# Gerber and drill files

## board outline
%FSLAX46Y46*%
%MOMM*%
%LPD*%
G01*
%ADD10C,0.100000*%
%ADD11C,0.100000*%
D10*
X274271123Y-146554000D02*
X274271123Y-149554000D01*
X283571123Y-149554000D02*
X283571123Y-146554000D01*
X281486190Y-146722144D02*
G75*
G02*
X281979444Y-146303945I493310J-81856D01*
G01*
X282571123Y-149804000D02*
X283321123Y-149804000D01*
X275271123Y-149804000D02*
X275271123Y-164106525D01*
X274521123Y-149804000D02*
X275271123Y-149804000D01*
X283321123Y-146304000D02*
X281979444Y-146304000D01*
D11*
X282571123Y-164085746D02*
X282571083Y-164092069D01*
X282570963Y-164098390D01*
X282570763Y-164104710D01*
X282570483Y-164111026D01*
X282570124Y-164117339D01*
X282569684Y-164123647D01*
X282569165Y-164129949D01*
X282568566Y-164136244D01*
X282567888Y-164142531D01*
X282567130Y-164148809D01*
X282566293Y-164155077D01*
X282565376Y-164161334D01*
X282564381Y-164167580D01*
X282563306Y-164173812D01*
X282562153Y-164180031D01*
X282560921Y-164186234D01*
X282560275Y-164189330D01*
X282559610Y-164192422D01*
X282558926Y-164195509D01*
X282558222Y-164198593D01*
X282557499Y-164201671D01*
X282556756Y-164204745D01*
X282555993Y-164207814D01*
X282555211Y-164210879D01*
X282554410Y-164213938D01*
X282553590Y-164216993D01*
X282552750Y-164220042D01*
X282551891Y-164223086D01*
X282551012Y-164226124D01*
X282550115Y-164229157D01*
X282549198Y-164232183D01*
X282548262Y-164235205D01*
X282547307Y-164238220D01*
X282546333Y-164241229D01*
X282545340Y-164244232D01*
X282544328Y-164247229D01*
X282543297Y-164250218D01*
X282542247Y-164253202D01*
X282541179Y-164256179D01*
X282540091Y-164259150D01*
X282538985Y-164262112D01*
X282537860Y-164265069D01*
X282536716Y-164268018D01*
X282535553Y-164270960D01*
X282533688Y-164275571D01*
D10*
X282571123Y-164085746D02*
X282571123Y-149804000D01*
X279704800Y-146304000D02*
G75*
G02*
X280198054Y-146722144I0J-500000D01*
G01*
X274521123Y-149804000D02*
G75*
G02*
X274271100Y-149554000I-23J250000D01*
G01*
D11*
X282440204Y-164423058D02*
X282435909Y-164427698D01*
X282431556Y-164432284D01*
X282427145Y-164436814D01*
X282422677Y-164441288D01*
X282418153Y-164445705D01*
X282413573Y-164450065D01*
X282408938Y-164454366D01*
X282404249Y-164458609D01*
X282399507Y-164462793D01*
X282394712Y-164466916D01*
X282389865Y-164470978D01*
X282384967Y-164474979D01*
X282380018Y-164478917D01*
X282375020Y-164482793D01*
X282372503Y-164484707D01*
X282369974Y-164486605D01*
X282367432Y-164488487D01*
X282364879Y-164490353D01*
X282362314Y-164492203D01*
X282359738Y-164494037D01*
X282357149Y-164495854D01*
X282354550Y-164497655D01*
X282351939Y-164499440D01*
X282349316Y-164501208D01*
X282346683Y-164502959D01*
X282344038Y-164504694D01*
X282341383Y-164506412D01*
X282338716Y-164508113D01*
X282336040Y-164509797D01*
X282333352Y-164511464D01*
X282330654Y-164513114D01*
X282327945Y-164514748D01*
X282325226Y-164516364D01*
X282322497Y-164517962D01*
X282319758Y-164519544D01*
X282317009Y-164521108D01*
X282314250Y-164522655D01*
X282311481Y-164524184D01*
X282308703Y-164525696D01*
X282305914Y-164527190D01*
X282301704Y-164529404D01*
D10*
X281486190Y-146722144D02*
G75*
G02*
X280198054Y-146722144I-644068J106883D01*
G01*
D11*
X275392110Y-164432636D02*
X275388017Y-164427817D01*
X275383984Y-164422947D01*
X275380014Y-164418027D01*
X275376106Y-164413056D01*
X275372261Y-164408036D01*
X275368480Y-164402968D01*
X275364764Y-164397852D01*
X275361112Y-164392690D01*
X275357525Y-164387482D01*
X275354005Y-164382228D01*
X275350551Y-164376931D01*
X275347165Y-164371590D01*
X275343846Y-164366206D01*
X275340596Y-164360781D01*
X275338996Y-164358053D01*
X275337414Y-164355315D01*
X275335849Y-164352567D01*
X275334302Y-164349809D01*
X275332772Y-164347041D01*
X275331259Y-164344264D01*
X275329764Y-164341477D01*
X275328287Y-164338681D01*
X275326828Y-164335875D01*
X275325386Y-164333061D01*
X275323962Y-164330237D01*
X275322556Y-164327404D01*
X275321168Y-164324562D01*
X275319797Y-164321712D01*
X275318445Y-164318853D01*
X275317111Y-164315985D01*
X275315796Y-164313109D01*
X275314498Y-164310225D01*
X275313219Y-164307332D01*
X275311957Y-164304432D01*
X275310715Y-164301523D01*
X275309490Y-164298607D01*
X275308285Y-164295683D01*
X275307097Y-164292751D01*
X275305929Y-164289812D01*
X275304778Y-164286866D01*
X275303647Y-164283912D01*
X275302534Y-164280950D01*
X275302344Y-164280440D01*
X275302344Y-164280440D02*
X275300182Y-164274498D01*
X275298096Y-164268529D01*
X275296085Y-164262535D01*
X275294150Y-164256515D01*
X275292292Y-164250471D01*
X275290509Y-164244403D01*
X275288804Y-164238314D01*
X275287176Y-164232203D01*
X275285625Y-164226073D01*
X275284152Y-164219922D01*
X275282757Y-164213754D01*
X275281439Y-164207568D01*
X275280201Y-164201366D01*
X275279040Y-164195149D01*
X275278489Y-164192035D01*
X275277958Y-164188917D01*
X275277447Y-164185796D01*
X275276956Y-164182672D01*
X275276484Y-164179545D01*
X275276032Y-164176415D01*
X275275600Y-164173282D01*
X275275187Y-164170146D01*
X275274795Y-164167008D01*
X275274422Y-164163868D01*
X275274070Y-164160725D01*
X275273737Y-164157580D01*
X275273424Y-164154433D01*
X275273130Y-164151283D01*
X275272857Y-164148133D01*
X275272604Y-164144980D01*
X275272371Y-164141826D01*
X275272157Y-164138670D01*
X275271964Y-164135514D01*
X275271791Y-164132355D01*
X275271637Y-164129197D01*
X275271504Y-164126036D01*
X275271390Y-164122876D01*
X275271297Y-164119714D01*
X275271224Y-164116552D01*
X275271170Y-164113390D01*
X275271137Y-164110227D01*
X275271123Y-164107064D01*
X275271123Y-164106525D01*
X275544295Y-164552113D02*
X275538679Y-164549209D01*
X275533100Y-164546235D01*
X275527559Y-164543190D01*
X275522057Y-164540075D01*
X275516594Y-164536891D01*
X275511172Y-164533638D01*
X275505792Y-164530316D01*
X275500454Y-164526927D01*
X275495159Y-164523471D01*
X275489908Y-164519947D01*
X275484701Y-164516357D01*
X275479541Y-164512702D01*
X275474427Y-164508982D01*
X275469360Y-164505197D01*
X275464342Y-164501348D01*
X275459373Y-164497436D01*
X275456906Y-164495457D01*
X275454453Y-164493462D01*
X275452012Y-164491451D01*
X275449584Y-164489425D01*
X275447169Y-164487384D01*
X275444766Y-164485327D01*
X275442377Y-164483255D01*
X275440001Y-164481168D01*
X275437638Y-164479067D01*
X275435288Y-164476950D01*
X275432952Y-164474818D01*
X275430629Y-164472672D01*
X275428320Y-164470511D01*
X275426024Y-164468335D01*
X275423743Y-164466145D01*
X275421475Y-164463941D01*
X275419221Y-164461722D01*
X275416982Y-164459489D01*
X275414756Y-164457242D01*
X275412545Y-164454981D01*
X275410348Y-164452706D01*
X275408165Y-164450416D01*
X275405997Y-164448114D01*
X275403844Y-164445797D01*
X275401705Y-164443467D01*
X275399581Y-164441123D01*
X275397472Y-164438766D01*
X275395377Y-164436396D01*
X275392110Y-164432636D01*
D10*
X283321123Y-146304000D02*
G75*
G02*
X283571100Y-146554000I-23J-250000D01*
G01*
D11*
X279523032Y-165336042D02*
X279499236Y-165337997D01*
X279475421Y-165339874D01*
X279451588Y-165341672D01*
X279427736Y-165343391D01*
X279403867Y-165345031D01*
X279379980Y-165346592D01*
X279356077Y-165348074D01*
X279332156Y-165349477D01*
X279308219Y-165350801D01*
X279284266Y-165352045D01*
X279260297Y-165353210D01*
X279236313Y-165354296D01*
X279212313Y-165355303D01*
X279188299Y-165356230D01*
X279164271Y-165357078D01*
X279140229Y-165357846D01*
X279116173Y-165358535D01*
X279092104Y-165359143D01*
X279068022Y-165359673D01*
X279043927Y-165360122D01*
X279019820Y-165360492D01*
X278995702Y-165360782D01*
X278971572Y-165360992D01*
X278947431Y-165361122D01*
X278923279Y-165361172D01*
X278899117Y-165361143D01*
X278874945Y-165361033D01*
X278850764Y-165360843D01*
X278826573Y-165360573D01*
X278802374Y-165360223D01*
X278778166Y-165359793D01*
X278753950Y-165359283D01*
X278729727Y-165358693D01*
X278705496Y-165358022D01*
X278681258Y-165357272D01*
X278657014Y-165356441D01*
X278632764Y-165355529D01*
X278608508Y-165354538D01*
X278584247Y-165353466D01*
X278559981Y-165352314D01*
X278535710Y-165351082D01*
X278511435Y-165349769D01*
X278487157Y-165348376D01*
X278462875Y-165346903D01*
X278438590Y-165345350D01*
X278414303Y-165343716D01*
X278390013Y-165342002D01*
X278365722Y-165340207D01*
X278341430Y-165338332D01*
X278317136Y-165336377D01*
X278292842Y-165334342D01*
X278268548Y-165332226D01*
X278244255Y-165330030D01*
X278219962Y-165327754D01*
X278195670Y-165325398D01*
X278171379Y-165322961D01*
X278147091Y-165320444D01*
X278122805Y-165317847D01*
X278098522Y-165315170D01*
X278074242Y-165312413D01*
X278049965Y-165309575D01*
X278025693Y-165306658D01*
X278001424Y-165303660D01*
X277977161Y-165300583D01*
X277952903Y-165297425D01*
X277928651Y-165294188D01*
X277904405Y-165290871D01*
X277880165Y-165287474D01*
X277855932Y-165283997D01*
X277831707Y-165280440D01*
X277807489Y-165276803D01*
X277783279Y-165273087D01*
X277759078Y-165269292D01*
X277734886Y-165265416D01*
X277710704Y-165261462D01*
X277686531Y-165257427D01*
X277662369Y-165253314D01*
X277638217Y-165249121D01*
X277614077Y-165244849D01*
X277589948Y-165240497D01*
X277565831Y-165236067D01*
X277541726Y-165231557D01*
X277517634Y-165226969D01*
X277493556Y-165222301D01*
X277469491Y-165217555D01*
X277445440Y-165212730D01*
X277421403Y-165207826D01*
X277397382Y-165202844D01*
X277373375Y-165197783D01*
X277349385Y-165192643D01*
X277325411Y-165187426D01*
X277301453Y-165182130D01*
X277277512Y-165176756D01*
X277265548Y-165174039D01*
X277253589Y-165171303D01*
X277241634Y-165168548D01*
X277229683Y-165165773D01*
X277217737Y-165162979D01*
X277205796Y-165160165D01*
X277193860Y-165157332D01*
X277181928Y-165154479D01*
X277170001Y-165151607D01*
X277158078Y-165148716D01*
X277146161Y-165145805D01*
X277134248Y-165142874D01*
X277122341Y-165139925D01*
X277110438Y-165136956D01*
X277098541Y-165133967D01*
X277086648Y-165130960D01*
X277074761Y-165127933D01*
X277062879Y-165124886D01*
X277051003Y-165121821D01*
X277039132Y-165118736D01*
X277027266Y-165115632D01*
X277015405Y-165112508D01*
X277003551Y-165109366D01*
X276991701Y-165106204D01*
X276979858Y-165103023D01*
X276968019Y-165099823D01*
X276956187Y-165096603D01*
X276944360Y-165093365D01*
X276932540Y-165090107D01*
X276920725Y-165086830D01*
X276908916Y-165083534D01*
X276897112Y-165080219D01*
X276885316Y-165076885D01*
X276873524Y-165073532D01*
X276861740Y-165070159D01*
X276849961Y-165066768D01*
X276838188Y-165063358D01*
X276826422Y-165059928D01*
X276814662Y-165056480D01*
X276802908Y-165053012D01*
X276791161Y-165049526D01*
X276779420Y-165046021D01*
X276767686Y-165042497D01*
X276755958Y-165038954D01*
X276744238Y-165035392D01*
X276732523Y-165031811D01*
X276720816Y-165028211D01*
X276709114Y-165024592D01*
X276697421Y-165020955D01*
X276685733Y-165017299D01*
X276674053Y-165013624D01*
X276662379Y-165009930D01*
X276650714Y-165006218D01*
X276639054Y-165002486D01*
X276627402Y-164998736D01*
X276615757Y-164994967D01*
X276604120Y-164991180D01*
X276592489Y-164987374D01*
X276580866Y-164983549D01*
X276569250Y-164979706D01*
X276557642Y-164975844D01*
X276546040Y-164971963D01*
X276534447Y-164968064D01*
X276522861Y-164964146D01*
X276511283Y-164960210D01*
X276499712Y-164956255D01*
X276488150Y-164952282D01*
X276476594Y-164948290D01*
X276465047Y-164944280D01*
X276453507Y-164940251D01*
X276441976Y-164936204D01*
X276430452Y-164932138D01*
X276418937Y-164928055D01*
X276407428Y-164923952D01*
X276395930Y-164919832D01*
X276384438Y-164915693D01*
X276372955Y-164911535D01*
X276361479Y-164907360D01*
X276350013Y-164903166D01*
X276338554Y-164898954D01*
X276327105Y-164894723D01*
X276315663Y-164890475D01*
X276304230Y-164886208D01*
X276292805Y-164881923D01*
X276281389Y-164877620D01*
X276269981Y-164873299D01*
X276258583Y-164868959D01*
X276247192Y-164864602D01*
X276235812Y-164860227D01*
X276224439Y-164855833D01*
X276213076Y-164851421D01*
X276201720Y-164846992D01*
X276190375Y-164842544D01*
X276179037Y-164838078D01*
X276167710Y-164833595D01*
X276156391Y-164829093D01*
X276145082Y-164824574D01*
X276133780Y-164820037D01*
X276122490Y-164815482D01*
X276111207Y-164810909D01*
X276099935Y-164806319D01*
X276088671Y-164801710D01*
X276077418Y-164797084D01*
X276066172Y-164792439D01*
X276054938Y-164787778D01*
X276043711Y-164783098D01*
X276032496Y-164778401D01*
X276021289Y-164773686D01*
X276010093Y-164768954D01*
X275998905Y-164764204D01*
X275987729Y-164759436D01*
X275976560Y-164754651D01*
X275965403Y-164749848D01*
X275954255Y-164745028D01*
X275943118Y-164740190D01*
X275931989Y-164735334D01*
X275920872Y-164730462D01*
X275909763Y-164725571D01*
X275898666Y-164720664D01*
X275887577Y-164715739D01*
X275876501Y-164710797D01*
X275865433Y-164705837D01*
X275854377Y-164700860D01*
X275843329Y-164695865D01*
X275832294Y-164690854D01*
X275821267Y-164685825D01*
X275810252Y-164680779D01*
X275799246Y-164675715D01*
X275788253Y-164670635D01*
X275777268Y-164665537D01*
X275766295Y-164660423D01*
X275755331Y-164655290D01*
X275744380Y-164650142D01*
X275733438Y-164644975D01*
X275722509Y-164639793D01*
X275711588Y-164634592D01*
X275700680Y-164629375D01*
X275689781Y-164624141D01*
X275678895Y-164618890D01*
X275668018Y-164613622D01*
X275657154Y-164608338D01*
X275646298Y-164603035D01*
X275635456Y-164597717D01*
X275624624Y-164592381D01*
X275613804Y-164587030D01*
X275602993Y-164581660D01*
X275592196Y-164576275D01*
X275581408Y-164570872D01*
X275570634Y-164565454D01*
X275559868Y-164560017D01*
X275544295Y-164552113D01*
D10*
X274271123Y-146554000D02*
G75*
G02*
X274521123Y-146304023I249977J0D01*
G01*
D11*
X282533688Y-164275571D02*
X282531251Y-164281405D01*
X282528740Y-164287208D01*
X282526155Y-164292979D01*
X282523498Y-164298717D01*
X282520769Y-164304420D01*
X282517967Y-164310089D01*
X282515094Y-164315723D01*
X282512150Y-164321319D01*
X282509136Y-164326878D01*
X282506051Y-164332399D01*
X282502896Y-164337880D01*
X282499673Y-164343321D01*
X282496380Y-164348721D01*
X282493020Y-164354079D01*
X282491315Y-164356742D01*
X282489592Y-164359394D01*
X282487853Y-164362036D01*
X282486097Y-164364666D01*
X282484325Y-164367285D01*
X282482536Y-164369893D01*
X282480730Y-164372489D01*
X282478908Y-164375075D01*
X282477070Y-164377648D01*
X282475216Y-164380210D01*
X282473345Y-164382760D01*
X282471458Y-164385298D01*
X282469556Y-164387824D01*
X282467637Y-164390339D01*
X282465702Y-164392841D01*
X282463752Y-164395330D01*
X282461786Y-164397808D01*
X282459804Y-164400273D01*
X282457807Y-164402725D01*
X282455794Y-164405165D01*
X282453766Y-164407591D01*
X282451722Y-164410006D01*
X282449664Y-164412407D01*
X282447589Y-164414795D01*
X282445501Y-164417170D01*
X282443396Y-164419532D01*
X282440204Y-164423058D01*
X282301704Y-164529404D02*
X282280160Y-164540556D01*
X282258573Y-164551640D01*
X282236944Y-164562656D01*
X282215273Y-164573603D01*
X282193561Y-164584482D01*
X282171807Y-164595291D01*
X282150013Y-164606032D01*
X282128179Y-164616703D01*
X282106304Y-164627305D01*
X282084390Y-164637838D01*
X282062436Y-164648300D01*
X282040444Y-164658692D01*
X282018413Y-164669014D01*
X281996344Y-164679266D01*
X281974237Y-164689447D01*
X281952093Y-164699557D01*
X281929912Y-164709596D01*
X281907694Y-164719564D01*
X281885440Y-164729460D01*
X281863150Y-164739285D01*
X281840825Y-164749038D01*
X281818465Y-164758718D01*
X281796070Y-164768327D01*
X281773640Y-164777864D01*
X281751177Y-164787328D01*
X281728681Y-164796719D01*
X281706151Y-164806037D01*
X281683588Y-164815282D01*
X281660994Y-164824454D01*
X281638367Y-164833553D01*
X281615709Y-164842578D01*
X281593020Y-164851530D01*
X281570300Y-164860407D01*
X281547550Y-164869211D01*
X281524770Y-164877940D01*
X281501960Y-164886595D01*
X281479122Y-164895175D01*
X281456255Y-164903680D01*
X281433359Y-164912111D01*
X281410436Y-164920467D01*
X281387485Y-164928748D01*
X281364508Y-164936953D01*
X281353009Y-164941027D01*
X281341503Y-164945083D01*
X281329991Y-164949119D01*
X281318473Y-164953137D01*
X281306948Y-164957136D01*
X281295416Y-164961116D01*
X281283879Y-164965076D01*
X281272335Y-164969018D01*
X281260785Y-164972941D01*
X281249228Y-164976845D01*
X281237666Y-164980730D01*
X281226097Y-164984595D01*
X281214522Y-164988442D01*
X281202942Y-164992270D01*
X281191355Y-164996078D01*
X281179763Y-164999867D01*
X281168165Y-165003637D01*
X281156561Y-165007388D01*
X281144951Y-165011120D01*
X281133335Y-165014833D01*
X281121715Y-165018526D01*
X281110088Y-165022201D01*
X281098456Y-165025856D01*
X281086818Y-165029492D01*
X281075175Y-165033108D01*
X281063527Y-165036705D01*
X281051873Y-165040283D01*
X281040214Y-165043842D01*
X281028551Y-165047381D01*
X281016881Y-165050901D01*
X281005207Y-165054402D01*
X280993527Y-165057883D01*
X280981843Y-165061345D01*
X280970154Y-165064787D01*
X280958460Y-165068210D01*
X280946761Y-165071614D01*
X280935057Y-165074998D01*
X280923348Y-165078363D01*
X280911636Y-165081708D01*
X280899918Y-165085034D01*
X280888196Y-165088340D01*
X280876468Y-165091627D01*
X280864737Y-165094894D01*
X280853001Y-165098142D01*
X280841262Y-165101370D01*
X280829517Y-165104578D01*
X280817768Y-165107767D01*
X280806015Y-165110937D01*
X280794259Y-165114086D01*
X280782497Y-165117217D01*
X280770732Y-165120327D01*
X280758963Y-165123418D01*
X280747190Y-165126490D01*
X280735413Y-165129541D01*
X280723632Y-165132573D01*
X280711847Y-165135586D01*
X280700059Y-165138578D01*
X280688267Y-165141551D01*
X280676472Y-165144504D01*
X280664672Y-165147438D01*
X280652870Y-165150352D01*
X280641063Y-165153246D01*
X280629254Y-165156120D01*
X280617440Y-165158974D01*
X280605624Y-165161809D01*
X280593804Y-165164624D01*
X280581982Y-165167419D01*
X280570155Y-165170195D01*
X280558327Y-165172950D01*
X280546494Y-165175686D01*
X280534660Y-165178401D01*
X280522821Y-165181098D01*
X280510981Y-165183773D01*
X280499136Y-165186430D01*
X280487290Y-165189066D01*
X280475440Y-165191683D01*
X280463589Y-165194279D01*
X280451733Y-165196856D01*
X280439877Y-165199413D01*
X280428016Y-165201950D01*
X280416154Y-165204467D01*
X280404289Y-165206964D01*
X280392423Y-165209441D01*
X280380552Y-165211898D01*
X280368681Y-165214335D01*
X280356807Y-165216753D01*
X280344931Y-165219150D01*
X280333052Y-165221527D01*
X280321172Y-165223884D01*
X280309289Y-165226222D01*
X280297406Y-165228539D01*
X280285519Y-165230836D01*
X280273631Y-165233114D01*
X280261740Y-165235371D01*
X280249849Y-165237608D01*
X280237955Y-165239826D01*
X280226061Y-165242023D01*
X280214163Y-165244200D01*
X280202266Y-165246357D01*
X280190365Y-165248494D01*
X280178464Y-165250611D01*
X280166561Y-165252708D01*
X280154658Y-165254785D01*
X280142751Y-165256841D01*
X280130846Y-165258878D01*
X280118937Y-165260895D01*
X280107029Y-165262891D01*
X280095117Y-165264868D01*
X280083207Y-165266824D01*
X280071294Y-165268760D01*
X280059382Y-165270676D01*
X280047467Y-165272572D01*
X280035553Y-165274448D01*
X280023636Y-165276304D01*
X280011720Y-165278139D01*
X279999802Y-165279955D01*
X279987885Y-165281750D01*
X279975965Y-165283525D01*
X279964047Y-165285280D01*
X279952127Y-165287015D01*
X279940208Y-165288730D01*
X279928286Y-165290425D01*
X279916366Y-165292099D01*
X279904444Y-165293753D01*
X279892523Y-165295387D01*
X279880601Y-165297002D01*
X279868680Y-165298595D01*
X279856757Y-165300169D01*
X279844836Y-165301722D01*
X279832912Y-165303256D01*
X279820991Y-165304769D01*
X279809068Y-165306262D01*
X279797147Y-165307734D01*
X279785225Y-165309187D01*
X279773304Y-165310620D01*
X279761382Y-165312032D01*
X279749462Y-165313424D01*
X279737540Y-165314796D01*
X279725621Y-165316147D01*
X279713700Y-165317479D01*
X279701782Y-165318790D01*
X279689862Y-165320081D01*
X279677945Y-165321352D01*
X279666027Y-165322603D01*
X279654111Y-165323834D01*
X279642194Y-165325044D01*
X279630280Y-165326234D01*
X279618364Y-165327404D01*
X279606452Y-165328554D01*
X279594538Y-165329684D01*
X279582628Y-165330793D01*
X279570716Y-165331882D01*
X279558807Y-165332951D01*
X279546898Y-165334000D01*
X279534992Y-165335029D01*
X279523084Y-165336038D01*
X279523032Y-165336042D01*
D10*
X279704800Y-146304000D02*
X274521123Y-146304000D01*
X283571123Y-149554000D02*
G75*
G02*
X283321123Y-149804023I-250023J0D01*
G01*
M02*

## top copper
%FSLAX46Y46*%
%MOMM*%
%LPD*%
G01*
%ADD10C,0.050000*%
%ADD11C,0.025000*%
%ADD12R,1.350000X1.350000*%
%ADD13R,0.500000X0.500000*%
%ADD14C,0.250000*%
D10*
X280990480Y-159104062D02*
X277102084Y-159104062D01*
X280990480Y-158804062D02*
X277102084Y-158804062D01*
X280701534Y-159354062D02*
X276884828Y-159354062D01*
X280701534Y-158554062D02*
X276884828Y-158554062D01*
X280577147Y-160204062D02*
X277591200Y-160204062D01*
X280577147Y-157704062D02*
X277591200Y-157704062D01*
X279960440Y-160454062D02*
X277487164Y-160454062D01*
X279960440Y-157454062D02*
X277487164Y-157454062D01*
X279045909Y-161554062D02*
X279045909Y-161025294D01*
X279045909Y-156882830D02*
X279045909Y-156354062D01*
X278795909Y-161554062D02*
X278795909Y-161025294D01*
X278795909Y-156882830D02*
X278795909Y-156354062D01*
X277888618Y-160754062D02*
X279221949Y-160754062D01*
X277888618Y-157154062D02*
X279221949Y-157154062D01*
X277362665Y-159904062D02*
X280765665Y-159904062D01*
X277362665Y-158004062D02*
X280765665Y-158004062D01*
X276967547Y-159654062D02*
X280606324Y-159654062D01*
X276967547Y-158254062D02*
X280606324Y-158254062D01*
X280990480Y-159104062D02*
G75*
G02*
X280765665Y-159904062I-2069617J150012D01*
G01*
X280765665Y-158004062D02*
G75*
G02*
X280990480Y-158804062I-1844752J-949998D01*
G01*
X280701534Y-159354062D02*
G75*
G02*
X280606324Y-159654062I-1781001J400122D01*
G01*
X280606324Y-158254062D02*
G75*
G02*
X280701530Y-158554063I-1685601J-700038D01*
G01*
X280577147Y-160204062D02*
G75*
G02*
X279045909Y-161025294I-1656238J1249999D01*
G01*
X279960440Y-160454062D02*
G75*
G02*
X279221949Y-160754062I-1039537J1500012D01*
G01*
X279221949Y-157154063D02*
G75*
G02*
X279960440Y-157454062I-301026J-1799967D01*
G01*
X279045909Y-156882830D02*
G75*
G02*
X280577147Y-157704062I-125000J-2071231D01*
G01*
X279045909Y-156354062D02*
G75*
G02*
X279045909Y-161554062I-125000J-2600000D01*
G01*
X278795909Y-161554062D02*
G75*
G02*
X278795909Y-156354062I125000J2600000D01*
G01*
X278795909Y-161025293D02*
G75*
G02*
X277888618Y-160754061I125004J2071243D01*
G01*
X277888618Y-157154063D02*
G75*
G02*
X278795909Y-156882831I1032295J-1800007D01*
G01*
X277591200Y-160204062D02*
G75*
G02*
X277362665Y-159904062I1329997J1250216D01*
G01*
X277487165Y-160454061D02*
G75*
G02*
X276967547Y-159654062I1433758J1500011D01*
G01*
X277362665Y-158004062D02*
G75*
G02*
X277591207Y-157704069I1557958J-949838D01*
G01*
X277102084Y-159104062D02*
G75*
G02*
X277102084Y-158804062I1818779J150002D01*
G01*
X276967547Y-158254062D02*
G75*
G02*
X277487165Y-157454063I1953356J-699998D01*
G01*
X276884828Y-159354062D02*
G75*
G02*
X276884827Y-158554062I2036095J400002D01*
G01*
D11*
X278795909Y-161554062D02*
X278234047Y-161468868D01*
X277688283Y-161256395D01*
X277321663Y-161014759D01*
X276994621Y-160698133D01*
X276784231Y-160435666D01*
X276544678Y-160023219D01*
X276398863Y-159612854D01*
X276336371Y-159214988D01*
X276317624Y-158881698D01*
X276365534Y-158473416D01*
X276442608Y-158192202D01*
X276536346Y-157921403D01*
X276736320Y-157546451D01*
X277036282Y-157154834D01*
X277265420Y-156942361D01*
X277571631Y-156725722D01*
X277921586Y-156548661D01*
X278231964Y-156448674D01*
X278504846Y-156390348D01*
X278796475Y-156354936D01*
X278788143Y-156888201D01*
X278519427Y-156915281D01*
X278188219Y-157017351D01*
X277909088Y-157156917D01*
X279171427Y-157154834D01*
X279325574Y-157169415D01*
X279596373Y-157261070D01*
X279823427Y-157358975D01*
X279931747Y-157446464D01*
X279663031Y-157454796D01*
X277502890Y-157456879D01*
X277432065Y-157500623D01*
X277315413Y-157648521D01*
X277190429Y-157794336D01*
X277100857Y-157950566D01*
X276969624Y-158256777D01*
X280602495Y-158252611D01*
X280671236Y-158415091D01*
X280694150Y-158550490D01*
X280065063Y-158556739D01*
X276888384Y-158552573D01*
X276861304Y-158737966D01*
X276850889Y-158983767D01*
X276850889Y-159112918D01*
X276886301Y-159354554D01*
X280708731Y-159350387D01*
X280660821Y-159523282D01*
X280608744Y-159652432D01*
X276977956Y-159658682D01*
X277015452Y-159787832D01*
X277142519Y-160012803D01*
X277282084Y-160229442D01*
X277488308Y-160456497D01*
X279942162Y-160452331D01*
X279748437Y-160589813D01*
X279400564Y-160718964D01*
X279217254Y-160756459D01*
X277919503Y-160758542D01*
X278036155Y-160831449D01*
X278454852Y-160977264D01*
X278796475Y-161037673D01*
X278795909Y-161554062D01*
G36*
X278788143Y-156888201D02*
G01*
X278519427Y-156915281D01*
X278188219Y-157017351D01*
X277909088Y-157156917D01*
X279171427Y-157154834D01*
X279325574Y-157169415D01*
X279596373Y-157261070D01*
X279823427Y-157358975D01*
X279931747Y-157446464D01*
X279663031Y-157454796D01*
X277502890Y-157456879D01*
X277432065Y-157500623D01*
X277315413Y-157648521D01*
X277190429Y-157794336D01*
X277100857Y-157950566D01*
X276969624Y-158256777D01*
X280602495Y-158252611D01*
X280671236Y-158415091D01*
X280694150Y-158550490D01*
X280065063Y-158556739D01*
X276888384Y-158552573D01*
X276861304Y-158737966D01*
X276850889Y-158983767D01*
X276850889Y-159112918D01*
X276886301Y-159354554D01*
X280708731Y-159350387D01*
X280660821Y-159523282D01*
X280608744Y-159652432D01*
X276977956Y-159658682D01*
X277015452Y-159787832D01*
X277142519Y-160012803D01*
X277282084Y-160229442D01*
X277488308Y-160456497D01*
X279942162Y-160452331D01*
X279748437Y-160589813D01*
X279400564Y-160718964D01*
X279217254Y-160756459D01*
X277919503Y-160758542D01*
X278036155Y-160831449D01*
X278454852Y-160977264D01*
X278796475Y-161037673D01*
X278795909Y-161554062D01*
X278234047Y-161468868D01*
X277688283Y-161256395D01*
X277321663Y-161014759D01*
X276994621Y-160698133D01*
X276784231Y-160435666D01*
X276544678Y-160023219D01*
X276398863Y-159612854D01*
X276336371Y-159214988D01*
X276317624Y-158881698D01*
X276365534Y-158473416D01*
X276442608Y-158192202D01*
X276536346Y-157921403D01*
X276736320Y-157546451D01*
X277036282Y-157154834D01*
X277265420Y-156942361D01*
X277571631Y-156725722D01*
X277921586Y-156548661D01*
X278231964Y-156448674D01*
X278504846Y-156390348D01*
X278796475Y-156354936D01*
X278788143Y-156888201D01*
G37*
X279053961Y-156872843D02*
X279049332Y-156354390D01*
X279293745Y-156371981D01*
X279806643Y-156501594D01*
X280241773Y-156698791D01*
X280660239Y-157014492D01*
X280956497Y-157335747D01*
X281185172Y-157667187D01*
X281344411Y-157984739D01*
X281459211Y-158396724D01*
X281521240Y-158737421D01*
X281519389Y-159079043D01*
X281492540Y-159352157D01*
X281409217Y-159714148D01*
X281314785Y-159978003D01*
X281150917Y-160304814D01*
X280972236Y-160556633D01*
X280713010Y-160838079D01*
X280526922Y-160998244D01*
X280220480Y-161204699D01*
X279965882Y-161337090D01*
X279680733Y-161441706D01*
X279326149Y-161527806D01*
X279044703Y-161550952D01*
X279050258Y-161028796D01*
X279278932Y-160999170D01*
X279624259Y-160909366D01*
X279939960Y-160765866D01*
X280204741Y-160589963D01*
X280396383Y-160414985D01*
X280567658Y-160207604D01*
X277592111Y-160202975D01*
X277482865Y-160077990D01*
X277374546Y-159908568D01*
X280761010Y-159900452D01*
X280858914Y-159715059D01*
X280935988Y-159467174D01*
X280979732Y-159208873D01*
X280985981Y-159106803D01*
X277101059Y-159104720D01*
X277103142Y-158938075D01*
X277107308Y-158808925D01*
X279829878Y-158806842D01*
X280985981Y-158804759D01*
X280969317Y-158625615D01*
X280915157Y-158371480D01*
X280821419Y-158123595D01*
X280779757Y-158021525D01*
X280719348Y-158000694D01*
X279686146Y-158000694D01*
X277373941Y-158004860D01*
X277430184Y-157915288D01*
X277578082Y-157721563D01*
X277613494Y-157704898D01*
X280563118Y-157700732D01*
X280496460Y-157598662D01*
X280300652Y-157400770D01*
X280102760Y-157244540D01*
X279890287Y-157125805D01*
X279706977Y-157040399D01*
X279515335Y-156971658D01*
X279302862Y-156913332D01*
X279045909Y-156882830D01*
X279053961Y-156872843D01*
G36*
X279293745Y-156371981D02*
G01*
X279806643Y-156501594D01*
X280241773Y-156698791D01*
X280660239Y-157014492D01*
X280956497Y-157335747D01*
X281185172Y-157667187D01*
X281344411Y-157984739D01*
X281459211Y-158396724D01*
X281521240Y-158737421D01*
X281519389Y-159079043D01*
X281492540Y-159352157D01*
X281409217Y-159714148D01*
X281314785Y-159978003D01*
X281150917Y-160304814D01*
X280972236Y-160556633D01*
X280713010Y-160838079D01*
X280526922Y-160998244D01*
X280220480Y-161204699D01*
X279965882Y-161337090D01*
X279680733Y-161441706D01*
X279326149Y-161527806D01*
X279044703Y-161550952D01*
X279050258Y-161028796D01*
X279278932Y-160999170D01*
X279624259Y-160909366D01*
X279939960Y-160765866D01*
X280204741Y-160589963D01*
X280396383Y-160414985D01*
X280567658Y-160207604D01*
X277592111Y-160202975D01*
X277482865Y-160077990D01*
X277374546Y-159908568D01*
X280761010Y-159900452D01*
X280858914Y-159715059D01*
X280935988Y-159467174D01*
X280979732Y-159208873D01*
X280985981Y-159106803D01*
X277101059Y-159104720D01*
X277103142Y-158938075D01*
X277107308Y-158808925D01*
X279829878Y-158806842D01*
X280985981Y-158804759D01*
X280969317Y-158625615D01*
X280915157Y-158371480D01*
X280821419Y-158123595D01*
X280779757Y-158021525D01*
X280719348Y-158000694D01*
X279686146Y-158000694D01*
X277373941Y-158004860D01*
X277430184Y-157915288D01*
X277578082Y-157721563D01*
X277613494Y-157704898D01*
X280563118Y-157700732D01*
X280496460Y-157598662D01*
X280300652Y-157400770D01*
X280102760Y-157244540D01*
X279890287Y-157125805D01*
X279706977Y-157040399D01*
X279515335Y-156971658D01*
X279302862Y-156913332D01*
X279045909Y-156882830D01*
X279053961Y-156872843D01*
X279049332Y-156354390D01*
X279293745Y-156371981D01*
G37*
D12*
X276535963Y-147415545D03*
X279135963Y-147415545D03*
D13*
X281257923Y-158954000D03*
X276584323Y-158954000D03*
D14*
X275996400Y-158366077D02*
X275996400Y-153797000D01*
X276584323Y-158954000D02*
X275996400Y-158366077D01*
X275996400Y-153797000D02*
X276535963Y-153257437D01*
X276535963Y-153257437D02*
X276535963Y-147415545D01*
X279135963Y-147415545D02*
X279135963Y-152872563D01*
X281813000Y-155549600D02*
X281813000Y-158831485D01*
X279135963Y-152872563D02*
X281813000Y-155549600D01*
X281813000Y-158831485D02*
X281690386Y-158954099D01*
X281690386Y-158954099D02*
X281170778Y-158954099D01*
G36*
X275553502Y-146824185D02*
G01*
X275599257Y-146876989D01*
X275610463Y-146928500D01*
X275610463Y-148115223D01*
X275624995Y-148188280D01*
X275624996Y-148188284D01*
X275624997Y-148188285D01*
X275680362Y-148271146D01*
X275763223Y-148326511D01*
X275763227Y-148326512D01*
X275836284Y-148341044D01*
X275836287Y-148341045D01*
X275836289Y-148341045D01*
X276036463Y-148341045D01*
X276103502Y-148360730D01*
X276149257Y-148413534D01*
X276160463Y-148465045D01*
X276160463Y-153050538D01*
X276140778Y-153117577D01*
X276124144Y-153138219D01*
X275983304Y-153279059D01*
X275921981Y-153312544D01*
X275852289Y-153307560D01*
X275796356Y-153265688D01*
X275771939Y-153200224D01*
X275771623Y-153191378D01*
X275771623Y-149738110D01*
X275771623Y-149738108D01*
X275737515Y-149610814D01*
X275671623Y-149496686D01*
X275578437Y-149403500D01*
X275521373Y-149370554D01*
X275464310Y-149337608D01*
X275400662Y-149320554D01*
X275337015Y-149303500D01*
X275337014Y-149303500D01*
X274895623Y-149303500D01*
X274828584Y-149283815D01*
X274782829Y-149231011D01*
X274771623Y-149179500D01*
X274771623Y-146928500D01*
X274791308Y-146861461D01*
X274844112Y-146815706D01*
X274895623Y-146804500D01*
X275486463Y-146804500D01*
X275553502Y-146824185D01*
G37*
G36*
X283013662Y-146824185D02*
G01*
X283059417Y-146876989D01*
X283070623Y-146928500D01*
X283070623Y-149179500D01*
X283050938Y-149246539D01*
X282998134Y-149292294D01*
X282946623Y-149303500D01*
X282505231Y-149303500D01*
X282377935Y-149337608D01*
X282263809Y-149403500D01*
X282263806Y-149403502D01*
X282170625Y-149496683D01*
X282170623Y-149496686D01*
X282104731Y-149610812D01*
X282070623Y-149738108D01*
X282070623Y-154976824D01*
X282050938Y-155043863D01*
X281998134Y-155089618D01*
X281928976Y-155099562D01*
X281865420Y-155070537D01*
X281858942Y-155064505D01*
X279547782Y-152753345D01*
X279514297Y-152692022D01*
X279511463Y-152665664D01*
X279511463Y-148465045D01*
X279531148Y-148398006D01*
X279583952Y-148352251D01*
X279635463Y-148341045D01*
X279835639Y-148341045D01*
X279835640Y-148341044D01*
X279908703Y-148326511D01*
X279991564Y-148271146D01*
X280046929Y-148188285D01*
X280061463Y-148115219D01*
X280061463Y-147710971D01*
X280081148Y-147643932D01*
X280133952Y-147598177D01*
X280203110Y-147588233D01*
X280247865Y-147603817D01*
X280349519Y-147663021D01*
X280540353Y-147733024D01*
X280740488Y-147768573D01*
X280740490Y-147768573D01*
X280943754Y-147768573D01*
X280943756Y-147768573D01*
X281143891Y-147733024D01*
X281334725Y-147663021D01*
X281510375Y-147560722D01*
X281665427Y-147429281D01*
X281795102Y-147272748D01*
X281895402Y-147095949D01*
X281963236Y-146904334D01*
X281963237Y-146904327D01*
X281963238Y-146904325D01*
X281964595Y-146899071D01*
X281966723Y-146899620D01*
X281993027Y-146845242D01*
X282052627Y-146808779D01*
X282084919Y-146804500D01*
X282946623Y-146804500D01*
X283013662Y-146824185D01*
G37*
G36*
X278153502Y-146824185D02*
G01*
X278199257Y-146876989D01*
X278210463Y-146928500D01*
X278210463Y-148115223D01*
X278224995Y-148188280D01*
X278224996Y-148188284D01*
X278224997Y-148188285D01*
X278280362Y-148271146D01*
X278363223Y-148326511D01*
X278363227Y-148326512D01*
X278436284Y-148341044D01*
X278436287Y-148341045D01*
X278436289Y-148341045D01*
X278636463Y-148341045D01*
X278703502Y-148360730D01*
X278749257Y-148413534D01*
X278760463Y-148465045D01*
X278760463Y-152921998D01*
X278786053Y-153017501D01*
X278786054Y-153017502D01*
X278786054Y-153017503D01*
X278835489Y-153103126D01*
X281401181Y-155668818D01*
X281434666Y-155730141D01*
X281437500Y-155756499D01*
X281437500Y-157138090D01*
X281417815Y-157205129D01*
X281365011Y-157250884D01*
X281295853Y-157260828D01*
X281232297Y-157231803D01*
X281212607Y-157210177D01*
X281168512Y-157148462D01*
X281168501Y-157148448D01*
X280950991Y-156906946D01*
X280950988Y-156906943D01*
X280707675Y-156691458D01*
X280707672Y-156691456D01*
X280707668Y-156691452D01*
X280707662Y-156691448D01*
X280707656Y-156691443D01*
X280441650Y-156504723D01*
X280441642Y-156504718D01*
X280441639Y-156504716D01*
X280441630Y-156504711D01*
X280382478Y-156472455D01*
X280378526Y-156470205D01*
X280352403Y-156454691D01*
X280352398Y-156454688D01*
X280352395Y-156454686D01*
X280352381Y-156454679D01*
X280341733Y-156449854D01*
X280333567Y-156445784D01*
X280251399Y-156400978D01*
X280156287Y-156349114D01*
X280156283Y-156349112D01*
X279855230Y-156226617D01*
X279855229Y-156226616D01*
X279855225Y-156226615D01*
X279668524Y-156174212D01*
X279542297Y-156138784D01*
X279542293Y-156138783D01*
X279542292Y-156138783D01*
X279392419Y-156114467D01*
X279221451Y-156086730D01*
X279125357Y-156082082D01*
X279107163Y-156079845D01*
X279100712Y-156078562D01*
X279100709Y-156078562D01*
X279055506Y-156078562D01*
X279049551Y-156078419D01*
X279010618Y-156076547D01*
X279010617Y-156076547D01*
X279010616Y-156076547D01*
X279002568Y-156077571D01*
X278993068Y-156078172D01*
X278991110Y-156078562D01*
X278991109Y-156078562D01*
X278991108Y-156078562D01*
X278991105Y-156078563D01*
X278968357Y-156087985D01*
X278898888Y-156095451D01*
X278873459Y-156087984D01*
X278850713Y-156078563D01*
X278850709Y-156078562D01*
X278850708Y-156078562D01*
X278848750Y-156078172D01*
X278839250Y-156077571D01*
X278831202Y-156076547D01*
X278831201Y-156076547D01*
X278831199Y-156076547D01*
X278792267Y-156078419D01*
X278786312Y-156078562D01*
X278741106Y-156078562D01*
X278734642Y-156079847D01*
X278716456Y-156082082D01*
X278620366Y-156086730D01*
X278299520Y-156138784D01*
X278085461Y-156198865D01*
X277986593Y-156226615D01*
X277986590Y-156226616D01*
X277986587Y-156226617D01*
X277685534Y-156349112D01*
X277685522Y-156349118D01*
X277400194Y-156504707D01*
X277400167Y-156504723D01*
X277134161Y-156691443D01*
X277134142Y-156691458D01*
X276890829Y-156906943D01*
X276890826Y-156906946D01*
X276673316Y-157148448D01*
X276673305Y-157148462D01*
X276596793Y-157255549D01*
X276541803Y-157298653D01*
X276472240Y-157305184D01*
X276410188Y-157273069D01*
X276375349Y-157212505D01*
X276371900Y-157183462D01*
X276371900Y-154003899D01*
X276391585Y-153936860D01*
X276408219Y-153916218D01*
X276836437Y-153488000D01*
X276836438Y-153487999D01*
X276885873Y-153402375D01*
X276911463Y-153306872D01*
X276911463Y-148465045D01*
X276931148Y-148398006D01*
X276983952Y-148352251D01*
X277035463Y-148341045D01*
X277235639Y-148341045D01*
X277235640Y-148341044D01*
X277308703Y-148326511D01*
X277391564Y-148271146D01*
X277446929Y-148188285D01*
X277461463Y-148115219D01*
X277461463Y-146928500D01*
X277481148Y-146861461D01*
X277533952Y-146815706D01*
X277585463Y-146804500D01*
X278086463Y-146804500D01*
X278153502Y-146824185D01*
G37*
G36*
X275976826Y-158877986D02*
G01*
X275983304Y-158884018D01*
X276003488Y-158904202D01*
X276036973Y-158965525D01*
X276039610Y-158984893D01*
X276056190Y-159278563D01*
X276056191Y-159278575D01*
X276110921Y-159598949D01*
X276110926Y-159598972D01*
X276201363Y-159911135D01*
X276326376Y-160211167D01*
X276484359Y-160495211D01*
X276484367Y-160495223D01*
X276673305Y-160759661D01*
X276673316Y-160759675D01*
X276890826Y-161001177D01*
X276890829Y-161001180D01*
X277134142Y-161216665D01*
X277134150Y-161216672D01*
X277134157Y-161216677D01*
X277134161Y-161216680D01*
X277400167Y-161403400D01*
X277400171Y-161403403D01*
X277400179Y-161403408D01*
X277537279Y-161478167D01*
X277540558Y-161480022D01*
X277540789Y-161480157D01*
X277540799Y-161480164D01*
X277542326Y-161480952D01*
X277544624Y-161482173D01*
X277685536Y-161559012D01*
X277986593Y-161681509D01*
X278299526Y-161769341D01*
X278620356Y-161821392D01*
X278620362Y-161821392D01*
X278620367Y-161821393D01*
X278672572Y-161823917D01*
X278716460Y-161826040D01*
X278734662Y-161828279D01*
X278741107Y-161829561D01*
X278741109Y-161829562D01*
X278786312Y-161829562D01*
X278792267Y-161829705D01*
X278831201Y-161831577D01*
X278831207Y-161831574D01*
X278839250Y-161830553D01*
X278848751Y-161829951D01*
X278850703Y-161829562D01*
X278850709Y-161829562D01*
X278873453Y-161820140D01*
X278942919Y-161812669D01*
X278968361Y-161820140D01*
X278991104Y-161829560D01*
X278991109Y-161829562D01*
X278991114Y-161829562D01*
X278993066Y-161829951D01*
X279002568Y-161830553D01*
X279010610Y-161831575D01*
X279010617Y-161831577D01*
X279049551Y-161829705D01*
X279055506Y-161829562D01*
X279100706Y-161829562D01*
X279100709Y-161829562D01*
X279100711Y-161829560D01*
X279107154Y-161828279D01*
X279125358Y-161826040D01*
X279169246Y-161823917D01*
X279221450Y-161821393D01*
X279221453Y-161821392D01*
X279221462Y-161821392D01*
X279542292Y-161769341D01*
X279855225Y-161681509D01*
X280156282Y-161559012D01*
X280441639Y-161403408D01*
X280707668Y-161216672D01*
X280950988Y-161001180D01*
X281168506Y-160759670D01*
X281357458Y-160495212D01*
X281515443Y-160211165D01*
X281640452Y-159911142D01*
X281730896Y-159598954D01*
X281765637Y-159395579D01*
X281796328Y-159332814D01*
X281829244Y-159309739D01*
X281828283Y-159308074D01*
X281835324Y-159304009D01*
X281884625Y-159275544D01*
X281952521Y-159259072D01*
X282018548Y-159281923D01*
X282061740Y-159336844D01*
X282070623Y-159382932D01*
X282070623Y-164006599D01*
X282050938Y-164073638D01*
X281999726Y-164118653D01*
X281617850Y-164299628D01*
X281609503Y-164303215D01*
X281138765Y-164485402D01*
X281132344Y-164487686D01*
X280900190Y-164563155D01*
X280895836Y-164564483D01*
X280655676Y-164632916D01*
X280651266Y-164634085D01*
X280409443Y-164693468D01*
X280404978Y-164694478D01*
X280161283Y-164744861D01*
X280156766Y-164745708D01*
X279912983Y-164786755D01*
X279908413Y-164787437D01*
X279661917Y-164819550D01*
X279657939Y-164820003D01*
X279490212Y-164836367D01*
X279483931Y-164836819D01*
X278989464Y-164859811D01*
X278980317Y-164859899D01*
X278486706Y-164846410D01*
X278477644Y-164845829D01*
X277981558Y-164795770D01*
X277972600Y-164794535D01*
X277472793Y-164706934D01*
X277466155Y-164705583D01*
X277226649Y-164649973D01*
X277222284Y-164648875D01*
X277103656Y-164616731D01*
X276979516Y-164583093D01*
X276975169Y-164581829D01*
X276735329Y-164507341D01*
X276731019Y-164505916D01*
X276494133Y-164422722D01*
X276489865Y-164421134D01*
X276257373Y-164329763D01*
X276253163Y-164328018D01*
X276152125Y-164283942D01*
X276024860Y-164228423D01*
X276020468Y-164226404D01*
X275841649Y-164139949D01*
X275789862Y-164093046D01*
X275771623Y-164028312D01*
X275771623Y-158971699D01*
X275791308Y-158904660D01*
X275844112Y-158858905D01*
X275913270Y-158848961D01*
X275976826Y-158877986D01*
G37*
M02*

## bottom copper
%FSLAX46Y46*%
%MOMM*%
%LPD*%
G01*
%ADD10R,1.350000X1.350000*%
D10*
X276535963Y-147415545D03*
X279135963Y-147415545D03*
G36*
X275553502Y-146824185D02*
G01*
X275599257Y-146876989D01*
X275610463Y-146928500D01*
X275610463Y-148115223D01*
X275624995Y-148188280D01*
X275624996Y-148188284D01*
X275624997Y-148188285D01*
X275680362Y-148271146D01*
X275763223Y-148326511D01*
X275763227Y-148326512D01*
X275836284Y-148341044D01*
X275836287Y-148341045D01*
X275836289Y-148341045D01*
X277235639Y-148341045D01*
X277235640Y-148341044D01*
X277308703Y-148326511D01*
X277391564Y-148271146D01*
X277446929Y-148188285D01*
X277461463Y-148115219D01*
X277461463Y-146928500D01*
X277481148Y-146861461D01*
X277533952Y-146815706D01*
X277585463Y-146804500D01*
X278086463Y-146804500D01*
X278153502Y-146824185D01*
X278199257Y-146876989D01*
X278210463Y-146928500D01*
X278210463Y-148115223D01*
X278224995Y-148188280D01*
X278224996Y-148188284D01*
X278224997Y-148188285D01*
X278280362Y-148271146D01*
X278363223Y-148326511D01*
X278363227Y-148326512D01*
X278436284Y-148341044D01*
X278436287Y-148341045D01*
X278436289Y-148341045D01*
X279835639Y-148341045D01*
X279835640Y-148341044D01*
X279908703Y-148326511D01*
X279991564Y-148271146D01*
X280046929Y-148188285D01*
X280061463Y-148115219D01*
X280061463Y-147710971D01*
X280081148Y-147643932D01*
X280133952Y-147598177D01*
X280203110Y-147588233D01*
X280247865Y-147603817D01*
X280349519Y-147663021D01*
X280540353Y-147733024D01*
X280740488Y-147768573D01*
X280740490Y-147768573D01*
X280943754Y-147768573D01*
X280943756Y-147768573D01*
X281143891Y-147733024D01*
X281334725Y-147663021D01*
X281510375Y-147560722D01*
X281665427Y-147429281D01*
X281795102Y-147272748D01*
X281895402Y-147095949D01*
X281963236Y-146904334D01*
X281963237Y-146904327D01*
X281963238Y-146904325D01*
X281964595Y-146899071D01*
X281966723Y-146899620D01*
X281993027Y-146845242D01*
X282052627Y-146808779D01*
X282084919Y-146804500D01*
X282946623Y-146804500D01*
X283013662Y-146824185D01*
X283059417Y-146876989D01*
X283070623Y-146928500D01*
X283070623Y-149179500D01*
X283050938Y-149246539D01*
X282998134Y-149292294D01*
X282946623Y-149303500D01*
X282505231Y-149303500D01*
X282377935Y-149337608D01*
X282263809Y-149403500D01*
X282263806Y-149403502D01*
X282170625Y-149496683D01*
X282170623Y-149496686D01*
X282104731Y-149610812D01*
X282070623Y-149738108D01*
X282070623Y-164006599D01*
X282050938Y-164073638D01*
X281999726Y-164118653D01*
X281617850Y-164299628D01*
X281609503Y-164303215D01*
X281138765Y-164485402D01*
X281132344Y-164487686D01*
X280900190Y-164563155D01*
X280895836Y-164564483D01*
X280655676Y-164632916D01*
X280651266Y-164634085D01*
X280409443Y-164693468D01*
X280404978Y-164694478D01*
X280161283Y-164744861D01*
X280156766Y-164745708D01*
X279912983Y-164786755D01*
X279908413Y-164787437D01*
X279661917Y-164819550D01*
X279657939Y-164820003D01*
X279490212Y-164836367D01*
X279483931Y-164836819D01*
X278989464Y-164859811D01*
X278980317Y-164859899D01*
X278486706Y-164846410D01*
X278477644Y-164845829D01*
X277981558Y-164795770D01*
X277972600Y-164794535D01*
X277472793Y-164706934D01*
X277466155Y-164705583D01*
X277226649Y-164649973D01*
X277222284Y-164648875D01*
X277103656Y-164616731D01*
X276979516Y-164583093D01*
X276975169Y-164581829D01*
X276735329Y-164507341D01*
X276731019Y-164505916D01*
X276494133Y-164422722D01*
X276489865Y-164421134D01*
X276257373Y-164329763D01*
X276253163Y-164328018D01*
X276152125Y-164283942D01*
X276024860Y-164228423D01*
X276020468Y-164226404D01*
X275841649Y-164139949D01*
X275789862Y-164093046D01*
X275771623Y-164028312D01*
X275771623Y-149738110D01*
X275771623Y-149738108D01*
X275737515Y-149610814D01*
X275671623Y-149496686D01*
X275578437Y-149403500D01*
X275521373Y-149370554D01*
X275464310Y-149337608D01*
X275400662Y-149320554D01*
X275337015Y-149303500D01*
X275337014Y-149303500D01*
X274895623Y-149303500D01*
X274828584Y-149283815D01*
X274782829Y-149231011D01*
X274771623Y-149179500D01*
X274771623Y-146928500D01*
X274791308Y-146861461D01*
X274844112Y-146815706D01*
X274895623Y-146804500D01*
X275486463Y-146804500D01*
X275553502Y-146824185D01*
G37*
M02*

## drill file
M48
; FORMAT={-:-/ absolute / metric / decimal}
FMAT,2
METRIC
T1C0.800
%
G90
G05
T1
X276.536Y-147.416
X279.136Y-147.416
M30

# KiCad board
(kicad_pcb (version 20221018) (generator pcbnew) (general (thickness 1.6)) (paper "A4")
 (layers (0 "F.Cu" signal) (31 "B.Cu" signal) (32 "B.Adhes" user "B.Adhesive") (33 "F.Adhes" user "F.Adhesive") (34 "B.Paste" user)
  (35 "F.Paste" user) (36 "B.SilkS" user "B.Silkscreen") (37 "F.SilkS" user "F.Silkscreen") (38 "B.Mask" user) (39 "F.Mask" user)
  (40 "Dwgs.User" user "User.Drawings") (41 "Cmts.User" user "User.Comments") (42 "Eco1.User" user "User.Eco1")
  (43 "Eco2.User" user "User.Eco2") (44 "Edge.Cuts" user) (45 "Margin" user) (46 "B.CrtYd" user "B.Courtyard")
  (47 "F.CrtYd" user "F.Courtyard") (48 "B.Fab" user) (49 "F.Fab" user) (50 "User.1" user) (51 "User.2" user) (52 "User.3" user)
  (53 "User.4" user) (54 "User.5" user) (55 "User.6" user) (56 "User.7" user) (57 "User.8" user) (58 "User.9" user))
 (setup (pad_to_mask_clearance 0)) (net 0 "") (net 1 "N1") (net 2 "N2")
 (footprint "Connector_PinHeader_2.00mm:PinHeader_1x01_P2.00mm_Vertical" (layer "F.Cu") (at 276.535963 147.415545)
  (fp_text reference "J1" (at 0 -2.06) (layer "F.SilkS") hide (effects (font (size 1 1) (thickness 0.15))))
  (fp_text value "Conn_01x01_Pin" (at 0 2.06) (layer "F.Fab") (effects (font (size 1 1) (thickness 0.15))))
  (pad "1" thru_hole rect (at 0 0) (size 1.35 1.35) (drill 0.8) (layers "*.Cu" "*.Mask") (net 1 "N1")))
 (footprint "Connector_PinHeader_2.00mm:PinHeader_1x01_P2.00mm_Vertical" (layer "F.Cu") (at 279.135963 147.415545)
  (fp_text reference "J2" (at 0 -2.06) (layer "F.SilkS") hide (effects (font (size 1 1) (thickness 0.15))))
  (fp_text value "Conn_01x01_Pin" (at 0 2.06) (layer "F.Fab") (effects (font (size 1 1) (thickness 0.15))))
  (pad "1" thru_hole rect (at 0 0) (size 1.35 1.35) (drill 0.8) (layers "*.Cu" "*.Mask") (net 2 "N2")))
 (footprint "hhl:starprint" (layer "F.Cu") (at 278.921123 158.954 180)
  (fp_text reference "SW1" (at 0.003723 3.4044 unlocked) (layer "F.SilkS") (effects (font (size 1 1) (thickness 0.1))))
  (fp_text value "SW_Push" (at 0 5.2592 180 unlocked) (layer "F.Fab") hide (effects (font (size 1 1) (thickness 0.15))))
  (fp_line (start -2.069357 -0.150062) (end 1.819039 -0.150062) (stroke (width 0.05) (type solid)) (layer "F.Cu"))
  (fp_line (start -2.069357 0.149938) (end 1.819039 0.149938) (stroke (width 0.05) (type solid)) (layer "F.Cu"))
  (fp_line (start -1.780411 -0.400062) (end 2.036295 -0.400062) (stroke (width 0.05) (type solid)) (layer "F.Cu"))
  (fp_line (start -1.780411 0.399938) (end 2.036295 0.399938) (stroke (width 0.05) (type solid)) (layer "F.Cu"))
  (fp_line (start -1.656024 -1.250062) (end 1.329923 -1.250062) (stroke (width 0.05) (type solid)) (layer "F.Cu"))
  (fp_line (start -1.656024 1.249938) (end 1.329923 1.249938) (stroke (width 0.05) (type solid)) (layer "F.Cu"))
  (fp_line (start -1.039317 -1.500062) (end 1.433959 -1.500062) (stroke (width 0.05) (type solid)) (layer "F.Cu"))
  (fp_line (start -1.039317 1.499938) (end 1.433959 1.499938) (stroke (width 0.05) (type solid)) (layer "F.Cu"))
  (fp_line (start -0.124786 -2.600062) (end -0.124786 -2.071294) (stroke (width 0.05) (type solid)) (layer "F.Cu"))
  (fp_line (start -0.124786 2.07117) (end -0.124786 2.599938) (stroke (width 0.05) (type solid)) (layer "F.Cu"))
  (fp_line (start 0.125214 -2.600062) (end 0.125214 -2.071294) (stroke (width 0.05) (type solid)) (layer "F.Cu"))
  (fp_line (start 0.125214 2.07117) (end 0.125214 2.599938) (stroke (width 0.05) (type solid)) (layer "F.Cu"))
  (fp_line (start 1.032505 -1.800062) (end -0.300826 -1.800062) (stroke (width 0.05) (type solid)) (layer "F.Cu"))
  (fp_line (start 1.032505 1.799938) (end -0.300826 1.799938) (stroke (width 0.05) (type solid)) (layer "F.Cu"))
  (fp_line (start 1.558458 -0.950062) (end -1.844542 -0.950062) (stroke (width 0.05) (type solid)) (layer "F.Cu"))
  (fp_line (start 1.558458 0.949938) (end -1.844542 0.949938) (stroke (width 0.05) (type solid)) (layer "F.Cu"))
  (fp_line (start 1.953576 -0.700062) (end -1.685201 -0.700062) (stroke (width 0.05) (type solid)) (layer "F.Cu"))
  (fp_line (start 1.953576 0.699938) (end -1.685201 0.699938) (stroke (width 0.05) (type solid)) (layer "F.Cu"))
  (fp_arc (start -2.069357 -0.150062) (mid -1.997406 -0.561431) (end -1.844542 -0.950062) (stroke (width 0.05) (type solid)) (layer "F.Cu"))
  (fp_arc (start -1.844542 0.949938) (mid -1.997407 0.561307) (end -2.069357 0.149938) (stroke (width 0.05) (type solid)) (layer "F.Cu"))
  (fp_arc (start -1.780411 -0.400062) (mid -1.739284 -0.552118) (end -1.685201 -0.700062) (stroke (width 0.05) (type solid)) (layer "F.Cu"))
  (fp_arc (start -1.685201 0.699938) (mid -1.739285 0.551994) (end -1.780411 0.399938) (stroke (width 0.05) (type solid)) (layer "F.Cu"))
  (fp_arc (start -1.656024 -1.250062) (mid -0.980504 -1.828673) (end -0.124786 -2.071294) (stroke (width 0.05) (type solid)) (layer "F.Cu"))
  (fp_arc (start -1.039317 -1.500062) (mid -0.68665 -1.690873) (end -0.300826 -1.800062) (stroke (width 0.05) (type solid)) (layer "F.Cu"))
  (fp_arc (start -0.300826 1.799937) (mid -0.68665 1.690749) (end -1.039316 1.499937) (stroke (width 0.05) (type solid)) (layer "F.Cu"))
  (fp_arc (start -0.124786 2.07117) (mid -0.980504 1.828549) (end -1.656024 1.249938) (stroke (width 0.05) (type solid)) (layer "F.Cu"))
  (fp_arc (start -0.124786 2.599938) (mid -2.602789 -0.000062) (end -0.124786 -2.600062) (stroke (width 0.05) (type solid)) (layer "F.Cu"))
  (fp_arc (start 0.125214 -2.600062) (mid 2.603217 -0.000062) (end 0.125214 2.599938) (stroke (width 0.05) (type solid)) (layer "F.Cu"))
  (fp_arc (start 0.125214 -2.071293) (mid 0.594539 -1.988126) (end 1.032505 -1.800061) (stroke (width 0.05) (type solid)) (layer "F.Cu"))
  (fp_arc (start 1.032505 1.799937) (mid 0.594539 1.988002) (end 0.125214 2.071169) (stroke (width 0.05) (type solid)) (layer "F.Cu"))
  (fp_arc (start 1.329923 -1.250062) (mid 1.451959 -1.10598) (end 1.558458 -0.950062) (stroke (width 0.05) (type solid)) (layer "F.Cu"))
  (fp_arc (start 1.433958 -1.500061) (mid 1.740364 -1.130327) (end 1.953577 -0.700062) (stroke (width 0.05) (type solid)) (layer "F.Cu"))
  (fp_arc (start 1.558458 0.949938) (mid 1.451962 1.105858) (end 1.329923 1.249938) (stroke (width 0.05) (type solid)) (layer "F.Cu"))
  (fp_arc (start 1.819039 -0.150062) (mid 1.825214 -0.000062) (end 1.819039 0.149938) (stroke (width 0.05) (type solid)) (layer "F.Cu"))
  (fp_arc (start 1.953576 0.699938) (mid 1.740364 1.130203) (end 1.433958 1.499937) (stroke (width 0.05) (type solid)) (layer "F.Cu"))
  (fp_arc (start 2.036295 -0.400062) (mid 2.075214 -0.000062) (end 2.036295 0.399938) (stroke (width 0.05) (type solid)) (layer "F.Cu"))
  (fp_poly
   (pts (xy 0.125214 -2.600062) (xy 0.687076 -2.514868) (xy 1.23284 -2.302395) (xy 1.59946 -2.060759) (xy 1.926502 -1.744133)
    (xy 2.136892 -1.481666) (xy 2.376445 -1.069219) (xy 2.52226 -0.658854) (xy 2.584752 -0.260988) (xy 2.603499 0.072302)
    (xy 2.555589 0.480584) (xy 2.478515 0.761798) (xy 2.384777 1.032597) (xy 2.184803 1.407549) (xy 1.884841 1.799166)
    (xy 1.655703 2.011639) (xy 1.349492 2.228278) (xy 0.999537 2.405339) (xy 0.689159 2.505326) (xy 0.416277 2.563652)
    (xy 0.124648 2.599064) (xy 0.13298 2.065799) (xy 0.401696 2.038719) (xy 0.732904 1.936649) (xy 1.012035 1.797083)
    (xy -0.250304 1.799166) (xy -0.404451 1.784585) (xy -0.67525 1.69293) (xy -0.902304 1.595025) (xy -1.010624 1.507536)
    (xy -0.741908 1.499204) (xy 1.418233 1.497121) (xy 1.489058 1.453377) (xy 1.60571 1.305479) (xy 1.730694 1.159664)
    (xy 1.820266 1.003434) (xy 1.951499 0.697223) (xy -1.681372 0.701389) (xy -1.750113 0.538909) (xy -1.773027 0.40351)
    (xy -1.14394 0.397261) (xy 2.032739 0.401427) (xy 2.059819 0.216034) (xy 2.070234 -0.029767) (xy 2.070234 -0.158918)
    (xy 2.034822 -0.400554) (xy -1.787608 -0.396387) (xy -1.739698 -0.569282) (xy -1.687621 -0.698432) (xy 1.943167 -0.704682)
    (xy 1.905671 -0.833832) (xy 1.778604 -1.058803) (xy 1.639039 -1.275442) (xy 1.432815 -1.502497) (xy -1.021039 -1.498331)
    (xy -0.827314 -1.635813) (xy -0.479441 -1.764964) (xy -0.296131 -1.802459) (xy 1.00162 -1.804542) (xy 0.884968 -1.877449)
    (xy 0.466271 -2.023264) (xy 0.124648 -2.083673))
   (stroke (width 0.025) (type solid)) (fill solid) (layer "F.Cu"))
  (fp_poly
   (pts (xy -0.132838 2.081157) (xy -0.128209 2.59961) (xy -0.372622 2.582019) (xy -0.88552 2.452406) (xy -1.32065 2.255209)
    (xy -1.739116 1.939508) (xy -2.035374 1.618253) (xy -2.264049 1.286813) (xy -2.423288 0.969261) (xy -2.538088 0.557276)
    (xy -2.600117 0.216579) (xy -2.598266 -0.125043) (xy -2.571417 -0.398157) (xy -2.488094 -0.760148) (xy -2.393662 -1.024003)
    (xy -2.229794 -1.350814) (xy -2.051113 -1.602633) (xy -1.791887 -1.884079) (xy -1.605799 -2.044244) (xy -1.299357 -2.250699)
    (xy -1.044759 -2.38309) (xy -0.75961 -2.487706) (xy -0.405026 -2.573806) (xy -0.12358 -2.596952) (xy -0.129135 -2.074796)
    (xy -0.357809 -2.04517) (xy -0.703136 -1.955366) (xy -1.018837 -1.811866) (xy -1.283618 -1.635963) (xy -1.47526 -1.460985)
    (xy -1.646535 -1.253604) (xy 1.329012 -1.248975) (xy 1.438258 -1.12399) (xy 1.546577 -0.954568) (xy -1.839887 -0.946452)
    (xy -1.937791 -0.761059) (xy -2.014865 -0.513174) (xy -2.058609 -0.254873) (xy -2.064858 -0.152803) (xy 1.820064 -0.15072)
    (xy 1.817981 0.015925) (xy 1.813815 0.145075) (xy -0.908755 0.147158) (xy -2.064858 0.149241) (xy -2.048194 0.328385)
    (xy -1.994034 0.58252) (xy -1.900296 0.830405) (xy -1.858634 0.932475) (xy -1.798225 0.953306) (xy -0.765023 0.953306)
    (xy 1.547182 0.94914) (xy 1.490939 1.038712) (xy 1.343041 1.232437) (xy 1.307629 1.249102) (xy -1.641995 1.253268)
    (xy -1.575337 1.355338) (xy -1.379529 1.55323) (xy -1.181637 1.70946) (xy -0.969164 1.828195) (xy -0.785854 1.913601)
    (xy -0.594212 1.982342) (xy -0.381739 2.040668) (xy -0.124786 2.07117))
   (stroke (width 0.025) (type solid)) (fill solid) (layer "F.Cu"))
  (pad "1" smd rect (at -2.3368 0 180) (size 0.5 0.5) (layers "F.Cu") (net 2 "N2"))
  (pad "2" smd rect (at 2.3368 0 180) (size 0.5 0.5) (layers "F.Cu") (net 1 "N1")))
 (gr_line (start 274.271123 146.554) (end 274.271123 149.554) (stroke (width 0.1) (type solid)) (layer "Edge.Cuts"))
 (gr_line (start 283.571123 149.554) (end 283.571123 146.554) (stroke (width 0.1) (type solid)) (layer "Edge.Cuts"))
 (gr_arc (start 281.48619 146.722144) (mid 281.656126 146.422611) (end 281.979444 146.304) (stroke (width 0.1) (type solid))
  (layer "Edge.Cuts"))
 (gr_line (start 282.571123 149.804) (end 283.321123 149.804) (stroke (width 0.1) (type solid)) (layer "Edge.Cuts"))
 (gr_line (start 275.271123 149.804) (end 275.271123 164.106525) (stroke (width 0.1) (type solid)) (layer "Edge.Cuts"))
 (gr_line (start 274.521123 149.804) (end 275.271123 149.804) (stroke (width 0.1) (type solid)) (layer "Edge.Cuts"))
 (gr_line (start 283.321123 146.304) (end 281.979444 146.304) (stroke (width 0.1) (type solid)) (layer "Edge.Cuts"))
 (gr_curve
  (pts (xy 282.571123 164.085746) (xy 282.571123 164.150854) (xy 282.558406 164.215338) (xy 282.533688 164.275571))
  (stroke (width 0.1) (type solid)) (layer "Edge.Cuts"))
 (gr_line (start 282.571123 164.085746) (end 282.571123 149.804) (stroke (width 0.1) (type solid)) (layer "Edge.Cuts"))
 (gr_arc (start 279.7048 146.304) (mid 280.028133 146.422594) (end 280.198054 146.722144) (stroke (width 0.1) (type solid))
  (layer "Edge.Cuts"))
 (gr_arc (start 274.521123 149.804) (mid 274.344346 149.730777) (end 274.271123 149.554) (stroke (width 0.1) (type solid))
  (layer "Edge.Cuts"))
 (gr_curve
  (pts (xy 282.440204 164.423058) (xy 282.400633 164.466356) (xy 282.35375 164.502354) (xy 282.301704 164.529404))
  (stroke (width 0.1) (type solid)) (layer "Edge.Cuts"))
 (gr_arc (start 281.48619 146.722144) (mid 280.842122 147.268137) (end 280.198054 146.722144) (stroke (width 0.1) (type solid))
  (layer "Edge.Cuts"))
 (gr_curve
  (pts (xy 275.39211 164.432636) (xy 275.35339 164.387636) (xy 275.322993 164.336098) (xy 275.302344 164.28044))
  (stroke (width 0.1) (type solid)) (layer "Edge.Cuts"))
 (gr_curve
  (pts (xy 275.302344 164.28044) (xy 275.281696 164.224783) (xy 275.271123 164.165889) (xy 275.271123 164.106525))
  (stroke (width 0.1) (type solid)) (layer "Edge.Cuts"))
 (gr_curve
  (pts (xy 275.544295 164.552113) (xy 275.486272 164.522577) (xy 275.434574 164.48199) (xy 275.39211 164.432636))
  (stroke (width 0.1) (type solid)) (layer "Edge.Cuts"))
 (gr_arc (start 283.321123 146.304) (mid 283.4979 146.377223) (end 283.571123 146.554) (stroke (width 0.1) (type solid)) (layer "Edge.Cuts"))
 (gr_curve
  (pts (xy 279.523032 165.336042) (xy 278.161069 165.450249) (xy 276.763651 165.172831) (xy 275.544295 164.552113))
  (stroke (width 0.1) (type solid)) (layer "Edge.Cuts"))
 (gr_arc (start 274.271123 146.554) (mid 274.344346 146.377223) (end 274.521123 146.304) (stroke (width 0.1) (type solid))
  (layer "Edge.Cuts"))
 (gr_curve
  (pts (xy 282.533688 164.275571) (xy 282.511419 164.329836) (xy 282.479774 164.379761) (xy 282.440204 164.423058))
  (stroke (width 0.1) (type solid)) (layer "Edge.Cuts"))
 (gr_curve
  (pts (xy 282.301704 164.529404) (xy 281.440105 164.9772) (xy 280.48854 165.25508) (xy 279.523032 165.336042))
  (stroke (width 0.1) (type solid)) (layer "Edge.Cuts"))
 (gr_line (start 279.7048 146.304) (end 274.521123 146.304) (stroke (width 0.1) (type solid)) (layer "Edge.Cuts"))
 (gr_arc (start 283.571123 149.554) (mid 283.4979 149.730777) (end 283.321123 149.804) (stroke (width 0.1) (type solid)) (layer "Edge.Cuts"))
 (segment (start 275.9964 158.366077) (end 275.9964 153.797) (width 0.25) (layer "F.Cu") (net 1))
 (segment (start 276.584323 158.954) (end 275.9964 158.366077) (width 0.25) (layer "F.Cu") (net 1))
 (segment (start 275.9964 153.797) (end 276.535963 153.257437) (width 0.25) (layer "F.Cu") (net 1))
 (segment (start 276.535963 153.257437) (end 276.535963 147.415545) (width 0.25) (layer "F.Cu") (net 1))
 (segment (start 279.135963 147.415545) (end 279.135963 152.872563) (width 0.25) (layer "F.Cu") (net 2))
 (segment (start 281.813 155.5496) (end 281.813 158.831485) (width 0.25) (layer "F.Cu") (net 2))
 (segment (start 279.135963 152.872563) (end 281.813 155.5496) (width 0.25) (layer "F.Cu") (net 2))
 (segment (start 281.813 158.831485) (end 281.690386 158.954099) (width 0.25) (layer "F.Cu") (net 2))
 (segment (start 281.690386 158.954099) (end 281.170778 158.954099) (width 0.25) (layer "F.Cu") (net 2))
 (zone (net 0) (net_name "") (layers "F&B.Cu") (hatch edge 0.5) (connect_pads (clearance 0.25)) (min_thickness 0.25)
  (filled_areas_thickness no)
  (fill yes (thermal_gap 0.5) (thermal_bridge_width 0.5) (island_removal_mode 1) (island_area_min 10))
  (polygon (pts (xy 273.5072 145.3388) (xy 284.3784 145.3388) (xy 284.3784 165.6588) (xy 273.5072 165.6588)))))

